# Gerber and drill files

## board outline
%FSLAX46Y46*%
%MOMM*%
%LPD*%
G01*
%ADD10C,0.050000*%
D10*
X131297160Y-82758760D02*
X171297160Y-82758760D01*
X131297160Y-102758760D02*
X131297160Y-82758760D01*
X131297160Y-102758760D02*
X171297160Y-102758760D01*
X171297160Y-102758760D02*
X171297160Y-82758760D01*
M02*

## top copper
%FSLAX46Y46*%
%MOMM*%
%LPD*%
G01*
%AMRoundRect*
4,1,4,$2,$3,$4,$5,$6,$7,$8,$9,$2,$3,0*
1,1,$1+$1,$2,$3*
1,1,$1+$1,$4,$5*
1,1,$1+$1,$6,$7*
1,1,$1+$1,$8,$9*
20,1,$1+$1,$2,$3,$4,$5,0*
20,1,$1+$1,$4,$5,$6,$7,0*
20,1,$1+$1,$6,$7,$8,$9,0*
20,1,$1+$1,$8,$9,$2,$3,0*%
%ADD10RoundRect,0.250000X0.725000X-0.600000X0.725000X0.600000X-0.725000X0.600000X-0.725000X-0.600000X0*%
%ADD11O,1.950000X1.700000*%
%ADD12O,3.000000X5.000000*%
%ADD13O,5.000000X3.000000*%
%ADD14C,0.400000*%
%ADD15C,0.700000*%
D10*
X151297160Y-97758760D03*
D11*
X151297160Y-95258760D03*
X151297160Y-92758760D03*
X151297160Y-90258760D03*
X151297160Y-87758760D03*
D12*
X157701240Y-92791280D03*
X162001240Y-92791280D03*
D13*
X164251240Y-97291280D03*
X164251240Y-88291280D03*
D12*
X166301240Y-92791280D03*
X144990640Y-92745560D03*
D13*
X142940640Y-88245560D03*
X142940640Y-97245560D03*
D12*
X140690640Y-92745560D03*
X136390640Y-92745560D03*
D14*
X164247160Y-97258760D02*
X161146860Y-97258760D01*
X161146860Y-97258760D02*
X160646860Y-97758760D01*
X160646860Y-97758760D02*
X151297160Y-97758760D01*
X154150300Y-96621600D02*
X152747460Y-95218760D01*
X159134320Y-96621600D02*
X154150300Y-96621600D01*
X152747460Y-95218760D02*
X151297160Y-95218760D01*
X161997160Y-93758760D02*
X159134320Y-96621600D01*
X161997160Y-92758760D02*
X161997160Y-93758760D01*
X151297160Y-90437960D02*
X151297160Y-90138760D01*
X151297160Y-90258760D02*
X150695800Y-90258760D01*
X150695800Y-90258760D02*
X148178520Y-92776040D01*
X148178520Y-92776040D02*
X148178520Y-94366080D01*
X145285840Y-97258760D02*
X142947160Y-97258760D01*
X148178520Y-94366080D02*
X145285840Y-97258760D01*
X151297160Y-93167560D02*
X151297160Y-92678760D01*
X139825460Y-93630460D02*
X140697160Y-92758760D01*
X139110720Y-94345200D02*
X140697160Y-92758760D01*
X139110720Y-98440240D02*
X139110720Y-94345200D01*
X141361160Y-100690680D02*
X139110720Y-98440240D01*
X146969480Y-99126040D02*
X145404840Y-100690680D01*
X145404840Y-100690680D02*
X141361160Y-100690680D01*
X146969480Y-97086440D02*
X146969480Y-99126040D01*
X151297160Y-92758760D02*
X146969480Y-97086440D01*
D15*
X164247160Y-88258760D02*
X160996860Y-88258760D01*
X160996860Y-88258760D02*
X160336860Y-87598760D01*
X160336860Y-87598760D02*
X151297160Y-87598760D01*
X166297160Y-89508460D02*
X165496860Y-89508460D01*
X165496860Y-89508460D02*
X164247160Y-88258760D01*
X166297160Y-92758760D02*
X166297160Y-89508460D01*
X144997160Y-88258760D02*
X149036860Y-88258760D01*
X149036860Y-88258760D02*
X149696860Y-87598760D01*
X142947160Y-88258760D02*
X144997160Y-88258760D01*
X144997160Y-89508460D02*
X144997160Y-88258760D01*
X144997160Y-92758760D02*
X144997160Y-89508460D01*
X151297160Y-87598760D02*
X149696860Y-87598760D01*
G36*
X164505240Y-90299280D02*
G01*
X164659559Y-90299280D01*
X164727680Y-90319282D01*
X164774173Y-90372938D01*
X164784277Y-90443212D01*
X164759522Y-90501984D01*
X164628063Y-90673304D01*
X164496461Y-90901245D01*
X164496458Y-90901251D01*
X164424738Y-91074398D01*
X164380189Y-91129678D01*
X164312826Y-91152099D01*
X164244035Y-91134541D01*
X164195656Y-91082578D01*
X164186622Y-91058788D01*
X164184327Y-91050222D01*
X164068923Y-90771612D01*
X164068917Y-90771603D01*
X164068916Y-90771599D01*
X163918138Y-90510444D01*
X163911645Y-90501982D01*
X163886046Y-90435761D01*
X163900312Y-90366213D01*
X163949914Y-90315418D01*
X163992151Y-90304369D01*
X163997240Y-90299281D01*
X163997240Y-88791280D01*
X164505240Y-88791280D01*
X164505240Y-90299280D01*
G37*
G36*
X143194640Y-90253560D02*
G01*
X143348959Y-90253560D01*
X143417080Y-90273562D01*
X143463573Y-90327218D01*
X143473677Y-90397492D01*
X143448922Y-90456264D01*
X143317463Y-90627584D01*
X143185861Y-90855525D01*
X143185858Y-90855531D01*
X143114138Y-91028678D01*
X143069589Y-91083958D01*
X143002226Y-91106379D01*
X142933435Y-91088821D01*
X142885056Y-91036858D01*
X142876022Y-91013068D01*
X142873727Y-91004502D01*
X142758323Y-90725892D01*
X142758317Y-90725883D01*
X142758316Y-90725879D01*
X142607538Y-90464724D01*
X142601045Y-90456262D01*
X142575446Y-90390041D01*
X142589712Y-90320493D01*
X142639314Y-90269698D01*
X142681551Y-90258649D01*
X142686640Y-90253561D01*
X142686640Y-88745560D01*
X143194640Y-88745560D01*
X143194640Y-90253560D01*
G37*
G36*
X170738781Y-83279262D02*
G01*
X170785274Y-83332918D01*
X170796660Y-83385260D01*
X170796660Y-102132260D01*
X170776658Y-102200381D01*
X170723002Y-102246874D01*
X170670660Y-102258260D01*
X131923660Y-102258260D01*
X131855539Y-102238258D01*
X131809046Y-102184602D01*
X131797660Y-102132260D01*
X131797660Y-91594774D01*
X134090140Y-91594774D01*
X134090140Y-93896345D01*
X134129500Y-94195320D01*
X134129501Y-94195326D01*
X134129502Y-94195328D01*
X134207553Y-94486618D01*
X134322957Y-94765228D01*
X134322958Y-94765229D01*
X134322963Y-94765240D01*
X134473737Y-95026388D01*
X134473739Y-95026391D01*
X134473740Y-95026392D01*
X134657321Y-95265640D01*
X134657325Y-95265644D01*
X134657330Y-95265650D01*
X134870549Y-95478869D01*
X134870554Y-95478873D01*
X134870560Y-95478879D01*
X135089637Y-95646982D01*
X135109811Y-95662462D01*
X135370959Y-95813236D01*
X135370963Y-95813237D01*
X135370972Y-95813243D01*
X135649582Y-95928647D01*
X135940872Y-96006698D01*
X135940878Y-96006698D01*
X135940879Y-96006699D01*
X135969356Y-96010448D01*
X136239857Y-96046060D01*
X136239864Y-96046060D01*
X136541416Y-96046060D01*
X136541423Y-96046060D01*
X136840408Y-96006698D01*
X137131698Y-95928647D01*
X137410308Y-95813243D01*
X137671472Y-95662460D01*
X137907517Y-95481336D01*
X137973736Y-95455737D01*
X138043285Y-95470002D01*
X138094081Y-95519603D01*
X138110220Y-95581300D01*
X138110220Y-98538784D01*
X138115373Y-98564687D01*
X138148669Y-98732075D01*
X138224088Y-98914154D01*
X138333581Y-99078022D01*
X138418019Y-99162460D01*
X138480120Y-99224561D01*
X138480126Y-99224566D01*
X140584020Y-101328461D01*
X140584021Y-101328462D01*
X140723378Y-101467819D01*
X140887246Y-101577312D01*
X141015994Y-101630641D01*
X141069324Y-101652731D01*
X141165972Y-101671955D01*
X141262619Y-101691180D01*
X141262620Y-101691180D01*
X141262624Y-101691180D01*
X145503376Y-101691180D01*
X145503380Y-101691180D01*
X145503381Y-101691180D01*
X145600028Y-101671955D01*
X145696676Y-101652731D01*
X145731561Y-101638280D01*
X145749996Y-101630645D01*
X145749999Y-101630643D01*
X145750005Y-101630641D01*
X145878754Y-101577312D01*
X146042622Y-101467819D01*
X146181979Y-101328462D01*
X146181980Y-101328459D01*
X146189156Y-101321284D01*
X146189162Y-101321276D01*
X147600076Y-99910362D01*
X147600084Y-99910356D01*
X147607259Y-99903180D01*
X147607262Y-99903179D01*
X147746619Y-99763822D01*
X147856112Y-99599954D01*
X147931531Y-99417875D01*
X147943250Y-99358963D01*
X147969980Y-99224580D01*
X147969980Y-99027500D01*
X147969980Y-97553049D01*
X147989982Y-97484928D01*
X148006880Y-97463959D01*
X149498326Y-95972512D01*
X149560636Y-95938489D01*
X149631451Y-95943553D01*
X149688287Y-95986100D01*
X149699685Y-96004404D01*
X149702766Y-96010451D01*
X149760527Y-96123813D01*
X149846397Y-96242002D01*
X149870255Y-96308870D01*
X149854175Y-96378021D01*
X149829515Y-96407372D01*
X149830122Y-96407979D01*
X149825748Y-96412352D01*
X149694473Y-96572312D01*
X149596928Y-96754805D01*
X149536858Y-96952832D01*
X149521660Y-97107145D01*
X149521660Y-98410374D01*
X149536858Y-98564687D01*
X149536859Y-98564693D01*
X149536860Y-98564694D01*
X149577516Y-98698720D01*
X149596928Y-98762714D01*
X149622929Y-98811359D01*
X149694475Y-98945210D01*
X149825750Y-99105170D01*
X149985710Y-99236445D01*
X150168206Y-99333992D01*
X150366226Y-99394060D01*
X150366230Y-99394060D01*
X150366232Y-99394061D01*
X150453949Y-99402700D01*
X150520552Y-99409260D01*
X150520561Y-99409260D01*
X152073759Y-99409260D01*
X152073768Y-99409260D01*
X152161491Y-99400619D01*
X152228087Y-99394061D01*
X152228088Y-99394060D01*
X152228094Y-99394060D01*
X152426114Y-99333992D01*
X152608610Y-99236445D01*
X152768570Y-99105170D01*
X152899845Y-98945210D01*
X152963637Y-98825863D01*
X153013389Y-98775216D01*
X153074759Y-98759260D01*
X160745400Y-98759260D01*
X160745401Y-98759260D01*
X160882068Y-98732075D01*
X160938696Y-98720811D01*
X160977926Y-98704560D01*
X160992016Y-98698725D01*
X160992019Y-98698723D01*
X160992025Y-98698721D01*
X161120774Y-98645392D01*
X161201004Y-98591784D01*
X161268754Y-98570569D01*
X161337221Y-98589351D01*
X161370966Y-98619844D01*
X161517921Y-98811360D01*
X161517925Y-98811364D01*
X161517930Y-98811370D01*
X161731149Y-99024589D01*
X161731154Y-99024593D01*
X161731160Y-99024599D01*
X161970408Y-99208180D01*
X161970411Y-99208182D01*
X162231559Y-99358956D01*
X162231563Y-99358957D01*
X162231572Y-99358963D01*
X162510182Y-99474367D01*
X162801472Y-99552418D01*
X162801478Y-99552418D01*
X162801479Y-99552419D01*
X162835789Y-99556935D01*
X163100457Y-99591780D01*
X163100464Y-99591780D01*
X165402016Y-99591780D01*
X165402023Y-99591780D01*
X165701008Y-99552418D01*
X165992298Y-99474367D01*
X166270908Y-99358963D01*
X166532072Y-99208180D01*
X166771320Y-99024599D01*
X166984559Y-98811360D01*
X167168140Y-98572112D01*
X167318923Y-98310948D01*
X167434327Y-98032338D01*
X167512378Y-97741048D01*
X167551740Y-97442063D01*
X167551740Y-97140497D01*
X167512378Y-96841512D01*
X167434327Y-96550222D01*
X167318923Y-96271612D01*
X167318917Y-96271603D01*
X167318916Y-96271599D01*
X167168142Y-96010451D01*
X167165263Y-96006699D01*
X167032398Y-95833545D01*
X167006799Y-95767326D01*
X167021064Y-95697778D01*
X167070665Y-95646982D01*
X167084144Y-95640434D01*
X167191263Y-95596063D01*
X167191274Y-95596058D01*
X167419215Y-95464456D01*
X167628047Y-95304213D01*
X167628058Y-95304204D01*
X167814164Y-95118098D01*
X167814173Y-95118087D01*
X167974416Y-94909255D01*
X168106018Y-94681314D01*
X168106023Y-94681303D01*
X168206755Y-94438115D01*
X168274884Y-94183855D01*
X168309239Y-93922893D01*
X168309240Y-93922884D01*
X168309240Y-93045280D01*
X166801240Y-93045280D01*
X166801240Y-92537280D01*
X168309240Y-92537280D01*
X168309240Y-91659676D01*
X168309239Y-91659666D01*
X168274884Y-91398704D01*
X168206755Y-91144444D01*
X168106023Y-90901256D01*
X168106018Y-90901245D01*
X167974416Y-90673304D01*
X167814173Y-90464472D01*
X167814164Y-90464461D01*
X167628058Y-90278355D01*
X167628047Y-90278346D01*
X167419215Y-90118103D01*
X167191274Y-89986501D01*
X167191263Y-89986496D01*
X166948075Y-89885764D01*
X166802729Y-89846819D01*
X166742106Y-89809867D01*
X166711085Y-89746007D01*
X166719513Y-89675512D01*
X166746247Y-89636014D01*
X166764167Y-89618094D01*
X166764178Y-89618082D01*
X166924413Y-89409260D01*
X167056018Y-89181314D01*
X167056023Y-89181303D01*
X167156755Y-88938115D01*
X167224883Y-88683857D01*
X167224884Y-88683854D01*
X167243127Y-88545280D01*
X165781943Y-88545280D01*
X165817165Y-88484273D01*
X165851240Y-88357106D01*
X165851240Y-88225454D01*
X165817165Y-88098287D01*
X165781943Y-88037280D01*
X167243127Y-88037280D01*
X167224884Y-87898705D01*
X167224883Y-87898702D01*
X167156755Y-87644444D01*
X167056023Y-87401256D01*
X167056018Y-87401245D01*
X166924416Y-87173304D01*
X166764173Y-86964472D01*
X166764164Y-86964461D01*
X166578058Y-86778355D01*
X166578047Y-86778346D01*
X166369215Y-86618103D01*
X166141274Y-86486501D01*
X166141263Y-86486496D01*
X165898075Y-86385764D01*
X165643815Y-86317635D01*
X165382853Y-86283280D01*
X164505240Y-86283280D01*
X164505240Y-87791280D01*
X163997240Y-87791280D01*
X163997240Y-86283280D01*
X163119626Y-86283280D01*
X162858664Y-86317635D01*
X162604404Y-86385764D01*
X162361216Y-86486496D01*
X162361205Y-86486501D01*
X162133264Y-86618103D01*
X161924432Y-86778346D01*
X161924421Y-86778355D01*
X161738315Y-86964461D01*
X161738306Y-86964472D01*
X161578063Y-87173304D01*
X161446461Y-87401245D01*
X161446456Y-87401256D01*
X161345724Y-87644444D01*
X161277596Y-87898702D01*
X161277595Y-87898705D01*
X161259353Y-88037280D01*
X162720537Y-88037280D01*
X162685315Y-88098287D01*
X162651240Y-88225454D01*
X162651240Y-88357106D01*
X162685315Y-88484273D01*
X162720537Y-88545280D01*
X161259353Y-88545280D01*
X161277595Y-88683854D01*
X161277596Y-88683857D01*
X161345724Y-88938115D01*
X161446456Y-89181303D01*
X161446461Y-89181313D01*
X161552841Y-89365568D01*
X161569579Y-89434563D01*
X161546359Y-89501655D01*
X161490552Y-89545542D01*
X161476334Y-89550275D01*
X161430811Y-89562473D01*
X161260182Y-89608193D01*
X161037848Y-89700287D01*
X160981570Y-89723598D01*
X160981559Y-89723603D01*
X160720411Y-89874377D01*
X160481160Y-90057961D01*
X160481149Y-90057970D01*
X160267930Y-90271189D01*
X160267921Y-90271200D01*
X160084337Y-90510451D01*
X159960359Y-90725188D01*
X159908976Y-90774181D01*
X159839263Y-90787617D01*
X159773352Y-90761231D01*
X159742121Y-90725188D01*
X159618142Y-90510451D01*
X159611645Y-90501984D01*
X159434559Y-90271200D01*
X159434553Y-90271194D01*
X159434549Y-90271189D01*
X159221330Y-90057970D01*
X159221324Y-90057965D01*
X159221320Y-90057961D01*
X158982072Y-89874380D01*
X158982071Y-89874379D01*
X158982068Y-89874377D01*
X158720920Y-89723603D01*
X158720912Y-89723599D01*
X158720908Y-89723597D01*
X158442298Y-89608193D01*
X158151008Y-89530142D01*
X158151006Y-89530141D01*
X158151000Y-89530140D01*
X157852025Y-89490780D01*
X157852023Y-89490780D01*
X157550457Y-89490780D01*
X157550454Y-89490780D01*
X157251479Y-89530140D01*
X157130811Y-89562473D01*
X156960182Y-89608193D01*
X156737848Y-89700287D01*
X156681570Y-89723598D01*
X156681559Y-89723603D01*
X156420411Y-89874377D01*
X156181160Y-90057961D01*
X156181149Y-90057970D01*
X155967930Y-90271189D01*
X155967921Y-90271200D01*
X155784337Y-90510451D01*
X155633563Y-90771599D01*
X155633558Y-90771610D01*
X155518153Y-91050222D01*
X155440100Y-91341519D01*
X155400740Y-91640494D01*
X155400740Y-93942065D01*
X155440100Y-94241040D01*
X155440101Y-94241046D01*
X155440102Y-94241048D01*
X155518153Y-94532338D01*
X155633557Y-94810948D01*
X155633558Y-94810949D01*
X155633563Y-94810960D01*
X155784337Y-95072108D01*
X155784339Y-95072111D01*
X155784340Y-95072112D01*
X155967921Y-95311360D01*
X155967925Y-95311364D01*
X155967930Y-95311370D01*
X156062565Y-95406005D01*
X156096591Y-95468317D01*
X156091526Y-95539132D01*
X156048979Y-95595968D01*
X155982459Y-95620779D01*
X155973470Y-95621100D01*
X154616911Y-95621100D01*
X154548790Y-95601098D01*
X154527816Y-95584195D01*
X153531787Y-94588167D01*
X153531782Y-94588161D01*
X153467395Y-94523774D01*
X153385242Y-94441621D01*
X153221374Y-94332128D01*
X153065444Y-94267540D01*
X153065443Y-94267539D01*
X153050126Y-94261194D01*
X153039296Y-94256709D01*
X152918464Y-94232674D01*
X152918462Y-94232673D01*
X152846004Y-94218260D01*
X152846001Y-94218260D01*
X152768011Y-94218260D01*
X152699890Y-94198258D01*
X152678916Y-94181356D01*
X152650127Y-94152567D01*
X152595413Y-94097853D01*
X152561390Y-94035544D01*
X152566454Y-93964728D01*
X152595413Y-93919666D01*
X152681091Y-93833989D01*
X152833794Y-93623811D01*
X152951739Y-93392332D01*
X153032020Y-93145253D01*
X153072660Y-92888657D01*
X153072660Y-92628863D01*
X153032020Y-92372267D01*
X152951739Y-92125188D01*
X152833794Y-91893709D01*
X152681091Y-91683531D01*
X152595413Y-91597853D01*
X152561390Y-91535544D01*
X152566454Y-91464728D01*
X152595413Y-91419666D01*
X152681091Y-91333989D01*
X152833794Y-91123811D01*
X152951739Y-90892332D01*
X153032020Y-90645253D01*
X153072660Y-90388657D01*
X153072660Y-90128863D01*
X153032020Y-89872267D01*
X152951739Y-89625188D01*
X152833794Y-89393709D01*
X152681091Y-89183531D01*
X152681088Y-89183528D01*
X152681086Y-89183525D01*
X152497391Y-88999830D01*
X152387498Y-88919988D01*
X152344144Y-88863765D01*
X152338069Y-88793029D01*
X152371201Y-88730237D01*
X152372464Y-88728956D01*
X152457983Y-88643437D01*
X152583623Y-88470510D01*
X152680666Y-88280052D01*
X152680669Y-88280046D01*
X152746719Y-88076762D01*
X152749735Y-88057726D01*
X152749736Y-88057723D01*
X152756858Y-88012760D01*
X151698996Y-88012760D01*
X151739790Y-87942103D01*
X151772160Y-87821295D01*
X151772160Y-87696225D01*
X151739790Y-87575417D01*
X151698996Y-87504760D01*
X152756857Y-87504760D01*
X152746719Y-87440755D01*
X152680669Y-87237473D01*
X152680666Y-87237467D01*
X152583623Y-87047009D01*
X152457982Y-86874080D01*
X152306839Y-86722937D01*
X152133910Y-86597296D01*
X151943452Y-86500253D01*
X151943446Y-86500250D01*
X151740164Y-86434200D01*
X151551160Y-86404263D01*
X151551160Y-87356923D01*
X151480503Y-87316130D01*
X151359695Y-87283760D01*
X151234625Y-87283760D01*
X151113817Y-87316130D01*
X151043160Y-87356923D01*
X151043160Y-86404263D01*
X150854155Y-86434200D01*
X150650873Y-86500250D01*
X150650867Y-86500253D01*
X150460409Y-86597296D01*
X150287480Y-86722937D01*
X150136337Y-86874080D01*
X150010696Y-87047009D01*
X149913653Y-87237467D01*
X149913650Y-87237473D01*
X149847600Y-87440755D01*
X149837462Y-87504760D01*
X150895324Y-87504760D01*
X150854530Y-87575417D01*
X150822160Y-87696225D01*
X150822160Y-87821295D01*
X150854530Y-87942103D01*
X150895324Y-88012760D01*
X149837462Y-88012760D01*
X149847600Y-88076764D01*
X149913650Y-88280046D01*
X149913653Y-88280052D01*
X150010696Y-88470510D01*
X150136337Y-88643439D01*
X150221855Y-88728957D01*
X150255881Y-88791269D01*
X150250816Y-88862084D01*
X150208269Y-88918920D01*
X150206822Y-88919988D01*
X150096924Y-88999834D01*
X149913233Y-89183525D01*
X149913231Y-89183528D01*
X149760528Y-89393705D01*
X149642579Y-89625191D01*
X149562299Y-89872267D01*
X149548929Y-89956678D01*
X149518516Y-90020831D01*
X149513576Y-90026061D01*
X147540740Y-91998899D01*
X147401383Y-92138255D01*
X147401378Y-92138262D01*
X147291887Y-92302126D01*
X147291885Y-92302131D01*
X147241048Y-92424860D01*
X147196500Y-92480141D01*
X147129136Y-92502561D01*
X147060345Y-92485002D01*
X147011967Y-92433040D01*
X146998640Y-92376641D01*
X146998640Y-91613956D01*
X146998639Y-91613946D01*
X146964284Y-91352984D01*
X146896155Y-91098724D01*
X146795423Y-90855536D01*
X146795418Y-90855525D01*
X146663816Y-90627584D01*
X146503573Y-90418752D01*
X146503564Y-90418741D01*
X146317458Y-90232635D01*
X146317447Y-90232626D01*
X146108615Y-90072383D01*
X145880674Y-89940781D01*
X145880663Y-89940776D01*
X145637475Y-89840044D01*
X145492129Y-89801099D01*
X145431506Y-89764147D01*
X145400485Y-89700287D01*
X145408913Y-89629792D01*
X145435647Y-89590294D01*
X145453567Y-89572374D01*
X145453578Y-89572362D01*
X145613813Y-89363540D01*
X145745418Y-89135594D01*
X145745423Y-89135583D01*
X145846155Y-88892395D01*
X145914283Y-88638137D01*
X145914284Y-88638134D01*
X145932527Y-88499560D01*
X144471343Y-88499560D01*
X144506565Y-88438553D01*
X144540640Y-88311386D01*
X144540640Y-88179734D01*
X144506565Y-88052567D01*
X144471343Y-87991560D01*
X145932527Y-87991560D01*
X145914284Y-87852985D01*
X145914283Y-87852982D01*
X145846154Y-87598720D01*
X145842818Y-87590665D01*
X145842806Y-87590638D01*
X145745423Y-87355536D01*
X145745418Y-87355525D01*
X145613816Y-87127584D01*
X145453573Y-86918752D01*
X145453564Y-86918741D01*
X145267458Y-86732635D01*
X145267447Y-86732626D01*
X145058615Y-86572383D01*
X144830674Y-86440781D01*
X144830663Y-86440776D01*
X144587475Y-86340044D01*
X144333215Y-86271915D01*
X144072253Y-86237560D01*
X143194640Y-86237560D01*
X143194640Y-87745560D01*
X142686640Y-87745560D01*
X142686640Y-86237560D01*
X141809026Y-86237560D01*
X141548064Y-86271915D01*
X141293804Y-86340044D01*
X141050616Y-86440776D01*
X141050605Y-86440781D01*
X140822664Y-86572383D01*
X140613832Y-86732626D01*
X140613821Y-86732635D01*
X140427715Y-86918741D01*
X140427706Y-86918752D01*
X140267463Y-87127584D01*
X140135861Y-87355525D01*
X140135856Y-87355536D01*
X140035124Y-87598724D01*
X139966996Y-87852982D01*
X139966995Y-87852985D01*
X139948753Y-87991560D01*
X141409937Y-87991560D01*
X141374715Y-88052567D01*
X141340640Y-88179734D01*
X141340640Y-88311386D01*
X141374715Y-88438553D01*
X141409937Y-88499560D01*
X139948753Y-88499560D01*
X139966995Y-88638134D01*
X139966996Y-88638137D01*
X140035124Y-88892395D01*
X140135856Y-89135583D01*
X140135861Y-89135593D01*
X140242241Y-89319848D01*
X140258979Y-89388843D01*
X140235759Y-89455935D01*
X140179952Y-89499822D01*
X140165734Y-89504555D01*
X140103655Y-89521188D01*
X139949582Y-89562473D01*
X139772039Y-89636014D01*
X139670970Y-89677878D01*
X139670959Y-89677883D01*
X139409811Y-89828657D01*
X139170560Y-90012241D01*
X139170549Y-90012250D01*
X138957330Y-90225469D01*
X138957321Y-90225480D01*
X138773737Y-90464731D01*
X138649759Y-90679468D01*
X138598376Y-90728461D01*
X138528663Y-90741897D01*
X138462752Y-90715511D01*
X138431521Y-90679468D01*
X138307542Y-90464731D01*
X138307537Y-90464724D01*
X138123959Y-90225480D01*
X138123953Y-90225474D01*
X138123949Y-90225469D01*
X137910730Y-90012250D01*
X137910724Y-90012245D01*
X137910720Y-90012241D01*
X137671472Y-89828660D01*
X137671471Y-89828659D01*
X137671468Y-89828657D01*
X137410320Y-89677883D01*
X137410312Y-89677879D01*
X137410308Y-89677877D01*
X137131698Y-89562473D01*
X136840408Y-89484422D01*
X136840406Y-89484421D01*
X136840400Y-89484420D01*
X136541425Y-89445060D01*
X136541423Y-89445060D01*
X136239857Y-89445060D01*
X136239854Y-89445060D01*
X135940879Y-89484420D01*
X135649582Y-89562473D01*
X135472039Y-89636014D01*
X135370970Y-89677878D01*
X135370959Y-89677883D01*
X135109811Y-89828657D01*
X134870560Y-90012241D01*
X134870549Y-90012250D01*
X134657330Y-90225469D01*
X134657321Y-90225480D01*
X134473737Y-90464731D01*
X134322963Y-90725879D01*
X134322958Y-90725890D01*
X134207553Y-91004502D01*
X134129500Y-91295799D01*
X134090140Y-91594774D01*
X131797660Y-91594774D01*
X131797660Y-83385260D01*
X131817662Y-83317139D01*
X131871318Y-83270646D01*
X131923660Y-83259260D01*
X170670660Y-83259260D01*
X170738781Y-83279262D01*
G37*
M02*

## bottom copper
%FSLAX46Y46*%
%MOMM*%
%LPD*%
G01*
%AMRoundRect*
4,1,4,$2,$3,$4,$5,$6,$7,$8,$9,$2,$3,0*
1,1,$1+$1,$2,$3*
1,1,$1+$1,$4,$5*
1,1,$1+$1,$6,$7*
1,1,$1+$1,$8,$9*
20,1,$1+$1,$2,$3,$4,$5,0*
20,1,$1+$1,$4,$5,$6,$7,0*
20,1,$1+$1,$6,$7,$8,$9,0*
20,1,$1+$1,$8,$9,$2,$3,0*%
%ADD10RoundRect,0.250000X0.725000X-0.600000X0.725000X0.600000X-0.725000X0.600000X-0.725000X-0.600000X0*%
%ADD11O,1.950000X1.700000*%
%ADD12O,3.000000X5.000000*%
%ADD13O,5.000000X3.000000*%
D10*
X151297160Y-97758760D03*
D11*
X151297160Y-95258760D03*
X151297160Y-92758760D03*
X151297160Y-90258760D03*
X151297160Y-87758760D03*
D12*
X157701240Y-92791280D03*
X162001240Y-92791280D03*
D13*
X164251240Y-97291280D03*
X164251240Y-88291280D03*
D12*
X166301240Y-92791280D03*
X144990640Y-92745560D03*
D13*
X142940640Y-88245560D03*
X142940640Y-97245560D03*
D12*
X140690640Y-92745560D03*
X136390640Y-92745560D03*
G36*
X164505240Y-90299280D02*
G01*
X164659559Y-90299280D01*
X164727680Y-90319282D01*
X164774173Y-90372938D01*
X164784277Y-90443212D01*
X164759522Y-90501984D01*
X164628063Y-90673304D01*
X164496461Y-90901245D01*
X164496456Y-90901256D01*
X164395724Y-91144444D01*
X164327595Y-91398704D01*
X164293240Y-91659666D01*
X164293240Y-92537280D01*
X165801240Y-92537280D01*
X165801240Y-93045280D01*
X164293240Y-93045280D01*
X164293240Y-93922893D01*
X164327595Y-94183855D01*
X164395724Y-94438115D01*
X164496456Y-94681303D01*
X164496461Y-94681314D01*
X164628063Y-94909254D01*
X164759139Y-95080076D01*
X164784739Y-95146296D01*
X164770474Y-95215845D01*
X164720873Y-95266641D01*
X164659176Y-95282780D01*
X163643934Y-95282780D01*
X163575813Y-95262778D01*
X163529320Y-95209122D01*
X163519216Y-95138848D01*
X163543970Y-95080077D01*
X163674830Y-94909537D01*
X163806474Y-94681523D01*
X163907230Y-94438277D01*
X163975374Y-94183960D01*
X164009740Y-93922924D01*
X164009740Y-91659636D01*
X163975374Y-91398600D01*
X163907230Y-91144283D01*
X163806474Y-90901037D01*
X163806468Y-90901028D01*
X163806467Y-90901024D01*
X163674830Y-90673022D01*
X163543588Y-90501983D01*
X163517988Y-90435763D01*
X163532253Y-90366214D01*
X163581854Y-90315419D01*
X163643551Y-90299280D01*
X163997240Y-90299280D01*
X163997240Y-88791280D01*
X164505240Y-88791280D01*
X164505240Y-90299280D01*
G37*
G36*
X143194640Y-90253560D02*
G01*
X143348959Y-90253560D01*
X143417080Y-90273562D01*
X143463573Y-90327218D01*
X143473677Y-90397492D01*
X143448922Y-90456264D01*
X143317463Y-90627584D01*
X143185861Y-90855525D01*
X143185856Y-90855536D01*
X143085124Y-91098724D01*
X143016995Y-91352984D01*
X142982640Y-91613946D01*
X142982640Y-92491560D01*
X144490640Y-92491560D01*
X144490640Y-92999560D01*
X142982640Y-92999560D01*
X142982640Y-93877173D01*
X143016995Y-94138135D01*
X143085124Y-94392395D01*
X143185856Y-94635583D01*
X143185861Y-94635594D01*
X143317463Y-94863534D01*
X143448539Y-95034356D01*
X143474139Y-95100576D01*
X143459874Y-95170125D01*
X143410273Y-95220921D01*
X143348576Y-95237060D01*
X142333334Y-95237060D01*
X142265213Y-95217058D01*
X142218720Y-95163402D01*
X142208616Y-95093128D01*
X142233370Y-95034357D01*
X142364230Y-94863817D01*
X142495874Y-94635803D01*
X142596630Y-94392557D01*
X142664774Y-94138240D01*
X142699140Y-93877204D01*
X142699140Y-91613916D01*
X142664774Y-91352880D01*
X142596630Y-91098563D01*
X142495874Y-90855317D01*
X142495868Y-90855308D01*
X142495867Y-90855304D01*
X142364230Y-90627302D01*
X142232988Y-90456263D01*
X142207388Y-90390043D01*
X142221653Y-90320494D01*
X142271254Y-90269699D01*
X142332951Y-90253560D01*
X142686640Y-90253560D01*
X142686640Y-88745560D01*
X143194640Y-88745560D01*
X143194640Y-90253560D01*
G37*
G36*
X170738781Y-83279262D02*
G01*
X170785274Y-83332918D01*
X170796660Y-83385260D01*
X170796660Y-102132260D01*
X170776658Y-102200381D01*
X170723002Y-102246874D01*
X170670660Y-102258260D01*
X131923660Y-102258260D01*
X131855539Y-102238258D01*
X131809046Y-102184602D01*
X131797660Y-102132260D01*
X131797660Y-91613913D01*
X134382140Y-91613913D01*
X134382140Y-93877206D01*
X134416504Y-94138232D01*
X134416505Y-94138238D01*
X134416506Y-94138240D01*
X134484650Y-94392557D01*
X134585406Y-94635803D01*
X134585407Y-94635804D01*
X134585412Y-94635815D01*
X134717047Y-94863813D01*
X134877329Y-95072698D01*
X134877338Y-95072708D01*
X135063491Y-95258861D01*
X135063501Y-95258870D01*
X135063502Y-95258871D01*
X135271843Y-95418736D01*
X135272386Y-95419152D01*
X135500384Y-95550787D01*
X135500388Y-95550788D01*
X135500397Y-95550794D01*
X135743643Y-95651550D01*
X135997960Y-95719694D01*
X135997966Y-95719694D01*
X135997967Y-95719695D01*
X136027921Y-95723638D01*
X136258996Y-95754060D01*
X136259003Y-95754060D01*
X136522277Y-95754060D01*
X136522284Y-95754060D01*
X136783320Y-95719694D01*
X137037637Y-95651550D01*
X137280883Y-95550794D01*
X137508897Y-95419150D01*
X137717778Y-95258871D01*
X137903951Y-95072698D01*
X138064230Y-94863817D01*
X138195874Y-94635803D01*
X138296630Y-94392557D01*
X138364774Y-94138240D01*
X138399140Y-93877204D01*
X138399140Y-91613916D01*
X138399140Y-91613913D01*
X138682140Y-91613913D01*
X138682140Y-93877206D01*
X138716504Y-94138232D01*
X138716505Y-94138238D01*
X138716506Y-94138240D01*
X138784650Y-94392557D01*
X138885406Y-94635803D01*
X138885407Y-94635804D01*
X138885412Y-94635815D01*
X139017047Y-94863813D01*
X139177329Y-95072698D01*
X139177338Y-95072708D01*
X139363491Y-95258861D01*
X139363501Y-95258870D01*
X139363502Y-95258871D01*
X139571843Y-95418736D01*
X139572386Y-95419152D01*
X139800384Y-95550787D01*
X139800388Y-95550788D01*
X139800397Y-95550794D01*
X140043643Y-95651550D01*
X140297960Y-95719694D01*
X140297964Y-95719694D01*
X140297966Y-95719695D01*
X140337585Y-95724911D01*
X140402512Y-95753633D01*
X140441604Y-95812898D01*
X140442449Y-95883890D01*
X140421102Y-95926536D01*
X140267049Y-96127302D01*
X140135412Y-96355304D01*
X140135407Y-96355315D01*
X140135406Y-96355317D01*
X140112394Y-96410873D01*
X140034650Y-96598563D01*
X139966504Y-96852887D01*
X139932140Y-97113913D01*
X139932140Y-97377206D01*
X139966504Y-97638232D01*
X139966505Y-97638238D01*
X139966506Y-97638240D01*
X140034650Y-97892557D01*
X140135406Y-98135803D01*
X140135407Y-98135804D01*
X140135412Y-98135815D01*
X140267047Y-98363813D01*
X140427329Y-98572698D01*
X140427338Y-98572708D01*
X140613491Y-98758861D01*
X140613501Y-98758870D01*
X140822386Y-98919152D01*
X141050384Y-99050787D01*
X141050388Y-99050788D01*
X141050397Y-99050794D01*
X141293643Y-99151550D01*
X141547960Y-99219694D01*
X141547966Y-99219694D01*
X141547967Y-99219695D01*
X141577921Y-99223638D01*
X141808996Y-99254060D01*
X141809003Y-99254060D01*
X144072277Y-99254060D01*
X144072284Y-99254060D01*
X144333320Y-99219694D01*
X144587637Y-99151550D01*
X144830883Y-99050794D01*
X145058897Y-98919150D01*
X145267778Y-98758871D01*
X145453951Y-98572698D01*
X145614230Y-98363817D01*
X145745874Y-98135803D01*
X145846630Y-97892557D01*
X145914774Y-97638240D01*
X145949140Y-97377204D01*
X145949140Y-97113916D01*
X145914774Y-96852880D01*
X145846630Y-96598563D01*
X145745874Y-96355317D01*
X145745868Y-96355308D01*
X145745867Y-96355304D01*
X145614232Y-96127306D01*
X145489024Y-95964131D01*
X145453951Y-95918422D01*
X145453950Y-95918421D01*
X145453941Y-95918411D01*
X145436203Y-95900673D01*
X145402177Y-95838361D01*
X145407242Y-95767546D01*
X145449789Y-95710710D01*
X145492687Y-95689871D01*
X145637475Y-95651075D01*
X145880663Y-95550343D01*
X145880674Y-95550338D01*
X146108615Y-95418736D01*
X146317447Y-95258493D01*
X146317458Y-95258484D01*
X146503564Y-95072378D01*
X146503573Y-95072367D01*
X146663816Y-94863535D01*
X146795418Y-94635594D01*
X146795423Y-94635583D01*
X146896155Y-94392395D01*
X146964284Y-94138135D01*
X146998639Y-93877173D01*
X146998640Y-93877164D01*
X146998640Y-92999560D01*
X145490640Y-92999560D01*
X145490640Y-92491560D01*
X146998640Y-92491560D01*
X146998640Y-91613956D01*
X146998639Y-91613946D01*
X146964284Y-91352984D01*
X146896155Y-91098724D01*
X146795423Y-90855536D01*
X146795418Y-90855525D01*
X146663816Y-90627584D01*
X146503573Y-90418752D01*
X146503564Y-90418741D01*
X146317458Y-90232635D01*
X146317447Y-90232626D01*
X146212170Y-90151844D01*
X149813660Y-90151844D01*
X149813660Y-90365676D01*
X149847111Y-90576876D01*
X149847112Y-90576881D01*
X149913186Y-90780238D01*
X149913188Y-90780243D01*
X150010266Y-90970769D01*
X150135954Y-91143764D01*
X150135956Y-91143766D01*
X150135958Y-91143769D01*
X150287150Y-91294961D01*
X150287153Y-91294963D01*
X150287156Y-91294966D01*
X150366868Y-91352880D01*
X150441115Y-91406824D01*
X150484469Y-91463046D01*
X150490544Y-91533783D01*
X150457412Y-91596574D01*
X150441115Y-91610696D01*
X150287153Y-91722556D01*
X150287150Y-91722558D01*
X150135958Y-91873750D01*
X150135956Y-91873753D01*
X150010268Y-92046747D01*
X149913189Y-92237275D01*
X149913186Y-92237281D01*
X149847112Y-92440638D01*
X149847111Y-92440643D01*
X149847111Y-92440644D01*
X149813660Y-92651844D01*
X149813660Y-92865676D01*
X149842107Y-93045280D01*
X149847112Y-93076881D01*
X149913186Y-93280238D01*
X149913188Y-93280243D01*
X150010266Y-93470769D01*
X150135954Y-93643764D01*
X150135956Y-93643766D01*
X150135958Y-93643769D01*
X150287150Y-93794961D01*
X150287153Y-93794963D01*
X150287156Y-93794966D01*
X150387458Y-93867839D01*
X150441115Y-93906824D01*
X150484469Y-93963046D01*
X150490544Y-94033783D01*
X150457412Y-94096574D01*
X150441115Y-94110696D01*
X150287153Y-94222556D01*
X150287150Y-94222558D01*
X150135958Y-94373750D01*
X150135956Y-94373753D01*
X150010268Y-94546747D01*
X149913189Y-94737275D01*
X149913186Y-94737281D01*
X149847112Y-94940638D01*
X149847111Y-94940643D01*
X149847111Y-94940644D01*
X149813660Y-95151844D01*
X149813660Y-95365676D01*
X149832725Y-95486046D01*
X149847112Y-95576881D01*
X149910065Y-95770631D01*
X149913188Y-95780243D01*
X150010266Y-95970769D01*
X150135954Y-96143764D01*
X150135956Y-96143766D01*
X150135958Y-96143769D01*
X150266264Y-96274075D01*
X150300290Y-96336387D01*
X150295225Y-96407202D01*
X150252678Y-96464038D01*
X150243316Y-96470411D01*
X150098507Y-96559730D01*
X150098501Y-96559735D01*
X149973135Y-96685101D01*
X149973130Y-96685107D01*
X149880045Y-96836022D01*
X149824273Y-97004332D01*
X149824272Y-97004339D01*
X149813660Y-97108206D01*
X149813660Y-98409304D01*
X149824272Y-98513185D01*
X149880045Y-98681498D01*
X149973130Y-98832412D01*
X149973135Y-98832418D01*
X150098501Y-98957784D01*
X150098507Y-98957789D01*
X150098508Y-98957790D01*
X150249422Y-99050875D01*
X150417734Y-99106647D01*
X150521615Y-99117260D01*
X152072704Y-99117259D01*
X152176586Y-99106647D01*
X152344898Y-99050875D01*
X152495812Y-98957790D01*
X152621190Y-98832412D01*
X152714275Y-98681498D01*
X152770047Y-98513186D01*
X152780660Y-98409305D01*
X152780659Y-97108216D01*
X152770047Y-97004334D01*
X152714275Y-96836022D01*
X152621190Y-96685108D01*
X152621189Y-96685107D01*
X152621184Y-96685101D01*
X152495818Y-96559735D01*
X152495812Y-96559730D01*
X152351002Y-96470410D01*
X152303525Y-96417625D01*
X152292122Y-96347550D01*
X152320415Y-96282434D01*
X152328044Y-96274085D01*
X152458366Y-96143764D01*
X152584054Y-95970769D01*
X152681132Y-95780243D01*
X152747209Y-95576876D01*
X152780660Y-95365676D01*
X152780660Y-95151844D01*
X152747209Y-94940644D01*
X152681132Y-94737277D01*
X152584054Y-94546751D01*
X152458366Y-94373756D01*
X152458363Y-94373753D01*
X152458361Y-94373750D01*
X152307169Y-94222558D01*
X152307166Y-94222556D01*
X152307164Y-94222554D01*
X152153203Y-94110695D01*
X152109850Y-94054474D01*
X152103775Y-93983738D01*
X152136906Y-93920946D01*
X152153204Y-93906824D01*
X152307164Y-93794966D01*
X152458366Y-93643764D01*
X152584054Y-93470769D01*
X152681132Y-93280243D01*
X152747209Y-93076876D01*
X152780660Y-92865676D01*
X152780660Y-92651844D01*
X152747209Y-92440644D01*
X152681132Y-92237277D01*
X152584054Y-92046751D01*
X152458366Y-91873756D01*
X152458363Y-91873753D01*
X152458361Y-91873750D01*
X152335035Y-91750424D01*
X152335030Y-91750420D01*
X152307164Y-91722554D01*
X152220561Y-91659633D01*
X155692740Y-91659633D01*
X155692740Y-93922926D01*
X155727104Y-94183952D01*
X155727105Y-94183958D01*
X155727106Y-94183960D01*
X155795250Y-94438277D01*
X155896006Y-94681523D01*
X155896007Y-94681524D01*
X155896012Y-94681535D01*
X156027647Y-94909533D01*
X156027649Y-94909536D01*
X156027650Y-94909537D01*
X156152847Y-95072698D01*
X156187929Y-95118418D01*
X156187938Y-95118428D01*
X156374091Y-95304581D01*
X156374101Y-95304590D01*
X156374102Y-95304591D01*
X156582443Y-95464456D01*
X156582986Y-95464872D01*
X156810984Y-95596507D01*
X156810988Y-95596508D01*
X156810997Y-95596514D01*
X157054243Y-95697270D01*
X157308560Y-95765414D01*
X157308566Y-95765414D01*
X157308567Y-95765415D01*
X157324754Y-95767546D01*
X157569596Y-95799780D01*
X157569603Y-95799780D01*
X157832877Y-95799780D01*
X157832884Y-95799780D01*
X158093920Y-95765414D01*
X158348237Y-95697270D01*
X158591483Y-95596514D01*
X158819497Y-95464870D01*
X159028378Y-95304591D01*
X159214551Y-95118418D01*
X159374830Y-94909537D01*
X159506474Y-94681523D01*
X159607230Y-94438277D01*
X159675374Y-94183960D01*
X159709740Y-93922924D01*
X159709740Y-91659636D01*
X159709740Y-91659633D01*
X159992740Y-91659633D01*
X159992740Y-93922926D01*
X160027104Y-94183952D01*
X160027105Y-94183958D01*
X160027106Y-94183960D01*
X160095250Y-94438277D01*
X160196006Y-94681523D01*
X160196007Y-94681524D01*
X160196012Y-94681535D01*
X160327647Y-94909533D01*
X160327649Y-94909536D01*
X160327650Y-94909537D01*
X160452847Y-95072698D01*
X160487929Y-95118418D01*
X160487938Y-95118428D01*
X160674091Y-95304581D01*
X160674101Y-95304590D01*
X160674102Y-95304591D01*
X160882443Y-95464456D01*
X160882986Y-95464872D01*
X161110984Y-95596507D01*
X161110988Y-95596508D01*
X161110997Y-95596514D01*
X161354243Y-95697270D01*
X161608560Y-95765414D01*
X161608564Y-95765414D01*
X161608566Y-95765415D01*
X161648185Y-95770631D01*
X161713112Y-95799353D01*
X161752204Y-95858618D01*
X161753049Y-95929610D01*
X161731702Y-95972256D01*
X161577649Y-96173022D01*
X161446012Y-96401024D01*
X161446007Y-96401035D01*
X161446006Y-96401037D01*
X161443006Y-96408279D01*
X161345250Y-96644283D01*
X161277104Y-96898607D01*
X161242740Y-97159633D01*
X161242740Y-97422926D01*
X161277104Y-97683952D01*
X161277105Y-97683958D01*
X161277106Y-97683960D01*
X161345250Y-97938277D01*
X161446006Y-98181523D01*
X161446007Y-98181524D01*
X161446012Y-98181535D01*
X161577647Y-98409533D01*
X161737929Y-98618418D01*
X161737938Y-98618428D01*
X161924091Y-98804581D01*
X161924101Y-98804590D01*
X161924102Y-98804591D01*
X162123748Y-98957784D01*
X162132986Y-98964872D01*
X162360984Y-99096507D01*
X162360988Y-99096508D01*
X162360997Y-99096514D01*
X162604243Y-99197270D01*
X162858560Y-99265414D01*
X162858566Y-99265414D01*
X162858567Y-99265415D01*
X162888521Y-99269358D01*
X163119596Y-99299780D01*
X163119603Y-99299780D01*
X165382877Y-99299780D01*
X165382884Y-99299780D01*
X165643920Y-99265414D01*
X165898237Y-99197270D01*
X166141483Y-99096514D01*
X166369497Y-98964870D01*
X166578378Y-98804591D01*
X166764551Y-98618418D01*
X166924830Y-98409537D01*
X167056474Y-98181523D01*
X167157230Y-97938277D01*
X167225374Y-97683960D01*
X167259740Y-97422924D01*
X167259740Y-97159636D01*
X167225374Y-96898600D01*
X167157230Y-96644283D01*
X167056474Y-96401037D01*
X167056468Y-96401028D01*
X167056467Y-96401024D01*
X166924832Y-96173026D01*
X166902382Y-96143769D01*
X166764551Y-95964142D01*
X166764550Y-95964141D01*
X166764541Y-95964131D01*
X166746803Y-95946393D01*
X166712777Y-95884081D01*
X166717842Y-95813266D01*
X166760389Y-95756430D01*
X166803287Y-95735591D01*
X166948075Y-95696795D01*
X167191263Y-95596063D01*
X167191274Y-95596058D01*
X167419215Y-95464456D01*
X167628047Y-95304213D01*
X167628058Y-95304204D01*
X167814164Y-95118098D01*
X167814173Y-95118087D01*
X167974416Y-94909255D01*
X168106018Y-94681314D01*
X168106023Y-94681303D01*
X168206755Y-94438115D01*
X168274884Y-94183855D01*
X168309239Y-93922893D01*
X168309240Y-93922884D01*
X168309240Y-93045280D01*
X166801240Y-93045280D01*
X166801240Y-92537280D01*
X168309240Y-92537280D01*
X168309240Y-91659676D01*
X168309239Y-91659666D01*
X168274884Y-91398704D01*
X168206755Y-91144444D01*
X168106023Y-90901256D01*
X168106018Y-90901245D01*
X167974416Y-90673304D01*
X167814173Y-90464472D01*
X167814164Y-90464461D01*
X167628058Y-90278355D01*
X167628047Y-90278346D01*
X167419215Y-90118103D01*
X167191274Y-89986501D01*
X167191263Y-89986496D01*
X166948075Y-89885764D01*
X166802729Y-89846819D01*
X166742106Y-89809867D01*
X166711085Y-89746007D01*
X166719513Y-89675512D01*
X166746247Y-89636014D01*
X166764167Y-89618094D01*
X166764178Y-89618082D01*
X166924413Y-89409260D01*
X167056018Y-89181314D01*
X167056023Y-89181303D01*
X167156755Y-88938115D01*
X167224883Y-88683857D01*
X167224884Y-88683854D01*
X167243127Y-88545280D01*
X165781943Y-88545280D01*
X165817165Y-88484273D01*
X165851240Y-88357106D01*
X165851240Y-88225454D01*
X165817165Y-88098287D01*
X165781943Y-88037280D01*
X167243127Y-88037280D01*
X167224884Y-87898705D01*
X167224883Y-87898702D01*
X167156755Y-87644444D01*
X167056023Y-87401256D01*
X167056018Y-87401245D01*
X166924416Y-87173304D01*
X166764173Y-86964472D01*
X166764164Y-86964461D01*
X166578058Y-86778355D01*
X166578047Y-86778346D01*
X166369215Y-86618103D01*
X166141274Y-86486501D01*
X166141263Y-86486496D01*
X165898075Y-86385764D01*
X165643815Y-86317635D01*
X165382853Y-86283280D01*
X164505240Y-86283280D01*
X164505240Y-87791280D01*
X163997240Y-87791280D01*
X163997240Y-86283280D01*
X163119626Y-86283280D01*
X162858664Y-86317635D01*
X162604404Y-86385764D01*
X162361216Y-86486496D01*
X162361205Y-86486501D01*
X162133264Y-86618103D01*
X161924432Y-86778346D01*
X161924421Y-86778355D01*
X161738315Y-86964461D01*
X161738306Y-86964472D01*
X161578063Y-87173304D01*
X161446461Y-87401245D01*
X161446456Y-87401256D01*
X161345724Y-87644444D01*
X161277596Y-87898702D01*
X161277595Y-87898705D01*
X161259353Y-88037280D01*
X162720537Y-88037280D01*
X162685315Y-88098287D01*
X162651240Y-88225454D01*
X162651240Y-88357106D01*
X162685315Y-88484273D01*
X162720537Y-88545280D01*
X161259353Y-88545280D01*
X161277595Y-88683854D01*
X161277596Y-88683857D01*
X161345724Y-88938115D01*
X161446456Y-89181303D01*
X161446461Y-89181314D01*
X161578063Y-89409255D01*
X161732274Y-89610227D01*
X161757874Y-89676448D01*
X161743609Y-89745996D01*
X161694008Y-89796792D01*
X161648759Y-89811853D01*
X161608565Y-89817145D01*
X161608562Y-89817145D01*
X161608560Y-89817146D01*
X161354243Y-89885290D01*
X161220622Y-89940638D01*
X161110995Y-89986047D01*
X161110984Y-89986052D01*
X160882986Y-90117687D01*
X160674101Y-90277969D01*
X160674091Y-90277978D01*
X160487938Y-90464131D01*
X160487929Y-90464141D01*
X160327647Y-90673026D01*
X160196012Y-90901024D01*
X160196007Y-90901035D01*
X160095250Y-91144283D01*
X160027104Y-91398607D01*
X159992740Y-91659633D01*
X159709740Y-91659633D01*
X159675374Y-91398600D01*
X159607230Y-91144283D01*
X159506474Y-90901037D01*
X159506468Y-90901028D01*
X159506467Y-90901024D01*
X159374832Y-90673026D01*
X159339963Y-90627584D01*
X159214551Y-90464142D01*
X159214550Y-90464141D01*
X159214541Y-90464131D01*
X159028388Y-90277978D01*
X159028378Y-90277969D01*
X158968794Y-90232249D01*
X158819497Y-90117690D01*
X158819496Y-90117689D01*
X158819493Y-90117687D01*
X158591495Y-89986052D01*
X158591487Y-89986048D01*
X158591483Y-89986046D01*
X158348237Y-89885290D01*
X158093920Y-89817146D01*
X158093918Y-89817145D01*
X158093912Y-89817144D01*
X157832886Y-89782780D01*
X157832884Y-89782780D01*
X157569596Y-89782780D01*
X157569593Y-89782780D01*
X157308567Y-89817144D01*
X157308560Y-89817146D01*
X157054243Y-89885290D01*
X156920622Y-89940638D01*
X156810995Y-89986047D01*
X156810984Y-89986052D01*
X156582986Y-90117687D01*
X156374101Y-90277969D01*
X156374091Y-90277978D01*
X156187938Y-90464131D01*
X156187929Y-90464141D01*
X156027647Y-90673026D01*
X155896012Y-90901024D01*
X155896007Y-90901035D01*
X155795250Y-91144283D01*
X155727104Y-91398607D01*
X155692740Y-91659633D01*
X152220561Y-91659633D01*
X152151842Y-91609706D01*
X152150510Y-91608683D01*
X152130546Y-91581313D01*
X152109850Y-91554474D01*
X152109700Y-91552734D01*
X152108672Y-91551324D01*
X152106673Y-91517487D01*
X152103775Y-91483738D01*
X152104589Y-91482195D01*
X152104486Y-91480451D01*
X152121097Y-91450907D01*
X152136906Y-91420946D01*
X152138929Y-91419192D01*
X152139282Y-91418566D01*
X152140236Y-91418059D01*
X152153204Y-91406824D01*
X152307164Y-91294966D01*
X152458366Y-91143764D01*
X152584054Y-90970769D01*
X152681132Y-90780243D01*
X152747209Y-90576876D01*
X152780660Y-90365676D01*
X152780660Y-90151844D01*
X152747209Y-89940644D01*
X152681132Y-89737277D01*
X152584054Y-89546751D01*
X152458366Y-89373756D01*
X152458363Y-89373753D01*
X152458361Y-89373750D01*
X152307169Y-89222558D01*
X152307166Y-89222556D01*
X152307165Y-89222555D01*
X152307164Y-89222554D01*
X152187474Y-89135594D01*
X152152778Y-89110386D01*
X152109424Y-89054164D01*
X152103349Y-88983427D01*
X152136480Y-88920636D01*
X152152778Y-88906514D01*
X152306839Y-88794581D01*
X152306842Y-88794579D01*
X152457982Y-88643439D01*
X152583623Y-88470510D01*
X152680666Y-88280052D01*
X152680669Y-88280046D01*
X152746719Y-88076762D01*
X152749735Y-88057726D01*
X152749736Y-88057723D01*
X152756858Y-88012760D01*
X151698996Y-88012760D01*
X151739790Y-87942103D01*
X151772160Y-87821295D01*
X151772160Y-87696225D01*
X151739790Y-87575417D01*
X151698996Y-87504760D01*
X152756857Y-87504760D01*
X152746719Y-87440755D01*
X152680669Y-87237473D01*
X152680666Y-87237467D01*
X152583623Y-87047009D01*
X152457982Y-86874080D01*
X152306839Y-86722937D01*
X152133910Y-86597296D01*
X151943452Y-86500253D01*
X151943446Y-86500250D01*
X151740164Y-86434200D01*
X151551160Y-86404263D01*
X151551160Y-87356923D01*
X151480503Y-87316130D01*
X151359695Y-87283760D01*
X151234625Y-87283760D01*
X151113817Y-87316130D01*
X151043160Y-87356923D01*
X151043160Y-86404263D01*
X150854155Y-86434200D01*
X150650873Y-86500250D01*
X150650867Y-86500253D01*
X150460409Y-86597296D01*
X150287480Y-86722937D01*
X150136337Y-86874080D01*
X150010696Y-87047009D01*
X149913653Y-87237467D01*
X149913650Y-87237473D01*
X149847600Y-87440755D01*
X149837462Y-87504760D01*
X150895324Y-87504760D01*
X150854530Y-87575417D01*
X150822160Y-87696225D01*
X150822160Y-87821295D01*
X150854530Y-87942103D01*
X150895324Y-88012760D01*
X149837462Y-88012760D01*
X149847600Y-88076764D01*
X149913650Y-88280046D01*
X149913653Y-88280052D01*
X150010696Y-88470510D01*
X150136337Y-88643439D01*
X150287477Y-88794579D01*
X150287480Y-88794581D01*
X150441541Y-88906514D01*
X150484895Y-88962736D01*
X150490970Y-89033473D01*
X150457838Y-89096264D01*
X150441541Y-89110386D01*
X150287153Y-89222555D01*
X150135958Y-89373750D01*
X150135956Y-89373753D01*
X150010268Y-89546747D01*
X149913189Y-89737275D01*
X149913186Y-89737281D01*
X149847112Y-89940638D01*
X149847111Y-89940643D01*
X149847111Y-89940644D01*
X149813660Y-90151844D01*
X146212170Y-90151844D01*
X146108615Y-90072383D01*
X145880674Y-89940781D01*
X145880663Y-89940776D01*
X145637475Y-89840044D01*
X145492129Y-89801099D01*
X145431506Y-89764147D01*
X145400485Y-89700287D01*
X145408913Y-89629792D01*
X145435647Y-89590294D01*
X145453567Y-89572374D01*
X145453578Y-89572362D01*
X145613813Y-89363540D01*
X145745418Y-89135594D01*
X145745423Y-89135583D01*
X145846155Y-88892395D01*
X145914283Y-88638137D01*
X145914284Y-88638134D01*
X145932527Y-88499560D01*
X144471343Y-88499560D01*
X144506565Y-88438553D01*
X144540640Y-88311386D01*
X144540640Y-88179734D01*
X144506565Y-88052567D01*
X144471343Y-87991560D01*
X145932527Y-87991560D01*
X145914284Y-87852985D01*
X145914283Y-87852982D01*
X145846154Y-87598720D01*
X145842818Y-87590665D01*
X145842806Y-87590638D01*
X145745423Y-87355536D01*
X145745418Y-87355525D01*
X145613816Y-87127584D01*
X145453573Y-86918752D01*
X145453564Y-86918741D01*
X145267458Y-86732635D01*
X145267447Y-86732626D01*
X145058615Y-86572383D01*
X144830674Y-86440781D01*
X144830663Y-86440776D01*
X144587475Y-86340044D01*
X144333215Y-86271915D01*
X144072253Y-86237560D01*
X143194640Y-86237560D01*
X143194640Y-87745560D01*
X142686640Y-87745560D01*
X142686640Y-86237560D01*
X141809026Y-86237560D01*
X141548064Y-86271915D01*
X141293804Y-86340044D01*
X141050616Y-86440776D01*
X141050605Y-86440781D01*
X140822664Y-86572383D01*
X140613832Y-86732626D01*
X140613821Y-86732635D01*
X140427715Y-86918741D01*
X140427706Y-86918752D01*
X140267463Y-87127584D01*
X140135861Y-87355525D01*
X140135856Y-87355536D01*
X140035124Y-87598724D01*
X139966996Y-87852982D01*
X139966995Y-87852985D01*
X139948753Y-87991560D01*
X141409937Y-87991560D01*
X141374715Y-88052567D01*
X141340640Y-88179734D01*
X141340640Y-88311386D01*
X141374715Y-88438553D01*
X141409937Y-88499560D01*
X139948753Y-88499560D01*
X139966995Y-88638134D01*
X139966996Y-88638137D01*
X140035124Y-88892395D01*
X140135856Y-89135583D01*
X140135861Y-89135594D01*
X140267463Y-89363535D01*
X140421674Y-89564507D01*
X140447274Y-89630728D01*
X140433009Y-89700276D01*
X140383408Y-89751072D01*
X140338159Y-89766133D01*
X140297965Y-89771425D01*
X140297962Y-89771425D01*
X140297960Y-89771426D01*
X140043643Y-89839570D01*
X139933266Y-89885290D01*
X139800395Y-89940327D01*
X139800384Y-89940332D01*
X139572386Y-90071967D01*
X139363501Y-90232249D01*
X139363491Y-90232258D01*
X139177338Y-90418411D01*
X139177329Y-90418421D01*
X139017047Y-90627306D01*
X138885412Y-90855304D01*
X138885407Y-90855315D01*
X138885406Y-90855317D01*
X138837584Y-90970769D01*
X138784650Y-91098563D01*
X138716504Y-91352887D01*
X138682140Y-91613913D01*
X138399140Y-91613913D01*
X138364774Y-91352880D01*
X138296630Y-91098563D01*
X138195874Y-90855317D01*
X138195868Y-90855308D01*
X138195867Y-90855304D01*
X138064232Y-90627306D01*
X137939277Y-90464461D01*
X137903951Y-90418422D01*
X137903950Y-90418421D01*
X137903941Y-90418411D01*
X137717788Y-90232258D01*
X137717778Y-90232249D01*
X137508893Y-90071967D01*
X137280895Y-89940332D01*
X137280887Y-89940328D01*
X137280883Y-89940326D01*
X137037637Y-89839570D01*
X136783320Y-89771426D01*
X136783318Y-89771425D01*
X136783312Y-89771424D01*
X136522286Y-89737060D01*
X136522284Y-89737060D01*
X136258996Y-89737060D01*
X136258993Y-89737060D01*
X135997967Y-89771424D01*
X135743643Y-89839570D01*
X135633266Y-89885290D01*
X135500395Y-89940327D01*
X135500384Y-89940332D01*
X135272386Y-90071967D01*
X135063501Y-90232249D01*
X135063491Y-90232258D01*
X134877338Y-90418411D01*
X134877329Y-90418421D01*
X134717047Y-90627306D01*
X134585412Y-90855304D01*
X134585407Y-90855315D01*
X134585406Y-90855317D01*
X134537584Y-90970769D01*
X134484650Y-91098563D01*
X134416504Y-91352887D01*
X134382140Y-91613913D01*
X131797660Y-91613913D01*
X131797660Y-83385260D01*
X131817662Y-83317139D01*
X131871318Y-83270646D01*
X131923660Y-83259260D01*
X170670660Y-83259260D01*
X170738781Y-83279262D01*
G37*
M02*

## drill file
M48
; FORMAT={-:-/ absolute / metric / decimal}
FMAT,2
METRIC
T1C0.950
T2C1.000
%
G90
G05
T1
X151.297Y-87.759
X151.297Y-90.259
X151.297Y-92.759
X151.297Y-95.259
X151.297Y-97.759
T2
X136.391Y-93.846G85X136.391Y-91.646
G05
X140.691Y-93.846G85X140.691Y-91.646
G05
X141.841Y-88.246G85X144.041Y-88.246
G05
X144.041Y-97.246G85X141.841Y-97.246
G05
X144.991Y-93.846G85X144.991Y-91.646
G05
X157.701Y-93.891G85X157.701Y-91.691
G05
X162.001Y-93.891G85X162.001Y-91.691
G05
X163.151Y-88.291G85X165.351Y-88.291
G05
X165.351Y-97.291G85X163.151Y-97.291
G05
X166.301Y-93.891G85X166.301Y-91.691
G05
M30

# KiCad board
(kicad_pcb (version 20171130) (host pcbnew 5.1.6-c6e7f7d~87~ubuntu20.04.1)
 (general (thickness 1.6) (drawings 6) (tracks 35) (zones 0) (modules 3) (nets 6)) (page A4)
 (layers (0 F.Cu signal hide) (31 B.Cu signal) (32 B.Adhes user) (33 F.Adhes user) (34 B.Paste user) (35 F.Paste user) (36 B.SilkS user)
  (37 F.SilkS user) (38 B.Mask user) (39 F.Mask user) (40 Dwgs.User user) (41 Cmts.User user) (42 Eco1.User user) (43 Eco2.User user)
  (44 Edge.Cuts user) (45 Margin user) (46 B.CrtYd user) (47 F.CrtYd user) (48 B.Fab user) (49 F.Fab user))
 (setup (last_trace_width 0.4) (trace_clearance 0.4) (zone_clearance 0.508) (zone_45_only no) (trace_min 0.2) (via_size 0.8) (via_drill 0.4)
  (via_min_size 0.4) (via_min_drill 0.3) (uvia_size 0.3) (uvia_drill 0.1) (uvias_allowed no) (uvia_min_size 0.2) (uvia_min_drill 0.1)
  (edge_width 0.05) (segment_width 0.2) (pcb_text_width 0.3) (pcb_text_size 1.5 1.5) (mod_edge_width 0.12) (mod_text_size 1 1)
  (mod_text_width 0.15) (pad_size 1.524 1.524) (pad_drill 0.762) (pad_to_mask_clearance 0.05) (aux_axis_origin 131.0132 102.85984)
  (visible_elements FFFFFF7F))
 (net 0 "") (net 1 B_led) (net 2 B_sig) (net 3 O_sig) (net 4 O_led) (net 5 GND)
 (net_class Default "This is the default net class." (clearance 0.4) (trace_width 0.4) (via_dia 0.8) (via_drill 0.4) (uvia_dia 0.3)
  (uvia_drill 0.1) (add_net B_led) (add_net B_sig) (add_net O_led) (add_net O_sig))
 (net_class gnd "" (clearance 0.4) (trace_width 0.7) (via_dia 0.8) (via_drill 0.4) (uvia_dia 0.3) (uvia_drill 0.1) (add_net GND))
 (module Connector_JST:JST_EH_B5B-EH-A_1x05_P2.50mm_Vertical (layer F.Cu) (at 151.29716 97.75876 90)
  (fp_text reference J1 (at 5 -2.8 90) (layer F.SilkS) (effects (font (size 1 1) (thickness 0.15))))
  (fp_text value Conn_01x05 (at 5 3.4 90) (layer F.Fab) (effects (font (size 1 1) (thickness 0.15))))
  (pad 1 thru_hole roundrect (at 0 0 90) (size 1.7 1.95) (drill 0.95) (layers *.Cu *.Mask) (roundrect_rratio 0.147059) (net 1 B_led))
  (pad 2 thru_hole oval (at 2.5 0 90) (size 1.7 1.95) (drill 0.95) (layers *.Cu *.Mask) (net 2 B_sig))
  (pad 3 thru_hole oval (at 5 0 90) (size 1.7 1.95) (drill 0.95) (layers *.Cu *.Mask) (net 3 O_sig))
  (pad 4 thru_hole oval (at 7.5 0 90) (size 1.7 1.95) (drill 0.95) (layers *.Cu *.Mask) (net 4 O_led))
  (pad 5 thru_hole oval (at 10 0 90) (size 1.7 1.95) (drill 0.95) (layers *.Cu *.Mask) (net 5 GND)))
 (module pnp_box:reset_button (layer F.Cu) (at 154.70124 92.79128 90)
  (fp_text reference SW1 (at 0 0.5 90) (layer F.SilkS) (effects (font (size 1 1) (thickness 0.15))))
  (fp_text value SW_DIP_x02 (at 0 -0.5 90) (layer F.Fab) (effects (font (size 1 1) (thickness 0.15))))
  (pad 0 thru_hole oval (at 0 3 90) (size 5 3) (drill oval 3.2 1) (layers *.Cu *.Mask))
  (pad 2 thru_hole oval (at 0 7.3 90) (size 5 3) (drill oval 3.2 1) (layers *.Cu *.Mask) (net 2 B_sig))
  (pad 1 thru_hole oval (at -4.5 9.55 180) (size 5 3) (drill oval 3.2 1) (layers *.Cu *.Mask) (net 1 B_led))
  (pad 4 thru_hole oval (at 4.5 9.55) (size 5 3) (drill oval 3.2 1) (layers *.Cu *.Mask) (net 5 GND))
  (pad 3 thru_hole oval (at 0 11.6 90) (size 5 3) (drill oval 3.2 1) (layers *.Cu *.Mask) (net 5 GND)))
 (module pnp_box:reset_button (layer F.Cu) (at 133.39064 92.74556 90)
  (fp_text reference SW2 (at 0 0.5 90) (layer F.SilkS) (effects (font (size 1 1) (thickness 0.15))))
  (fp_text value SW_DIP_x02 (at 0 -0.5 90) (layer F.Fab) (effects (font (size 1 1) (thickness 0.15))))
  (pad 3 thru_hole oval (at 0 11.6 90) (size 5 3) (drill oval 3.2 1) (layers *.Cu *.Mask) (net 5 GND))
  (pad 4 thru_hole oval (at 4.5 9.55) (size 5 3) (drill oval 3.2 1) (layers *.Cu *.Mask) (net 5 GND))
  (pad 1 thru_hole oval (at -4.5 9.55 180) (size 5 3) (drill oval 3.2 1) (layers *.Cu *.Mask) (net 4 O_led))
  (pad 2 thru_hole oval (at 0 7.3 90) (size 5 3) (drill oval 3.2 1) (layers *.Cu *.Mask) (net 3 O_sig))
  (pad 0 thru_hole oval (at 0 3 90) (size 5 3) (drill oval 3.2 1) (layers *.Cu *.Mask)))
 (gr_line (start 131.29716 82.75876) (end 171.29716 82.75876) (layer Edge.Cuts) (width 0.05))
 (gr_line (start 131.29716 102.75876) (end 131.29716 82.75876) (layer Edge.Cuts) (width 0.05))
 (gr_line (start 131.29716 102.75876) (end 171.29716 102.75876) (layer Edge.Cuts) (width 0.05))
 (gr_line (start 171.29716 102.75876) (end 171.29716 82.75876) (layer Edge.Cuts) (width 0.05))
 (segment (start 164.24716 97.25876) (end 161.14686 97.25876) (width 0.4) (layer F.Cu) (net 1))
 (segment (start 161.14686 97.25876) (end 160.64686 97.75876) (width 0.4) (layer F.Cu) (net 1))
 (segment (start 160.64686 97.75876) (end 151.29716 97.75876) (width 0.4) (layer F.Cu) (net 1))
 (segment (start 154.1503 96.6216) (end 152.74746 95.21876) (width 0.4) (layer F.Cu) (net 2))
 (segment (start 159.13432 96.6216) (end 154.1503 96.6216) (width 0.4) (layer F.Cu) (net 2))
 (segment (start 152.74746 95.21876) (end 151.29716 95.21876) (width 0.4) (layer F.Cu) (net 2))
 (segment (start 161.99716 93.75876) (end 159.13432 96.6216) (width 0.4) (layer F.Cu) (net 2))
 (segment (start 161.99716 92.75876) (end 161.99716 93.75876) (width 0.4) (layer F.Cu) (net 2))
 (segment (start 151.29716 90.43796) (end 151.29716 90.13876) (width 0.4) (layer F.Cu) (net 4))
 (segment (start 151.29716 90.25876) (end 150.6958 90.25876) (width 0.4) (layer F.Cu) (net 4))
 (segment (start 150.6958 90.25876) (end 148.17852 92.77604) (width 0.4) (layer F.Cu) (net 4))
 (segment (start 148.17852 92.77604) (end 148.17852 94.36608) (width 0.4) (layer F.Cu) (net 4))
 (segment (start 145.28584 97.25876) (end 142.94716 97.25876) (width 0.4) (layer F.Cu) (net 4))
 (segment (start 148.17852 94.36608) (end 145.28584 97.25876) (width 0.4) (layer F.Cu) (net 4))
 (segment (start 151.29716 93.16756) (end 151.29716 92.67876) (width 0.4) (layer F.Cu) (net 3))
 (segment (start 139.82546 93.63046) (end 140.69716 92.75876) (width 0.4) (layer F.Cu) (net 3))
 (segment (start 139.11072 94.3452) (end 140.69716 92.75876) (width 0.4) (layer F.Cu) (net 3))
 (segment (start 139.11072 98.44024) (end 139.11072 94.3452) (width 0.4) (layer F.Cu) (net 3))
 (segment (start 141.36116 100.69068) (end 139.11072 98.44024) (width 0.4) (layer F.Cu) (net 3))
 (segment (start 146.96948 99.12604) (end 145.40484 100.69068) (width 0.4) (layer F.Cu) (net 3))
 (segment (start 145.40484 100.69068) (end 141.36116 100.69068) (width 0.4) (layer F.Cu) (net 3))
 (segment (start 146.96948 97.08644) (end 146.96948 99.12604) (width 0.4) (layer F.Cu) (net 3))
 (segment (start 151.29716 92.75876) (end 146.96948 97.08644) (width 0.4) (layer F.Cu) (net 3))
 (segment (start 164.24716 88.25876) (end 160.99686 88.25876) (width 0.7) (layer F.Cu) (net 5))
 (segment (start 160.99686 88.25876) (end 160.33686 87.59876) (width 0.7) (layer F.Cu) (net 5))
 (segment (start 160.33686 87.59876) (end 151.29716 87.59876) (width 0.7) (layer F.Cu) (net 5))
 (segment (start 166.29716 89.50846) (end 165.49686 89.50846) (width 0.7) (layer F.Cu) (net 5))
 (segment (start 165.49686 89.50846) (end 164.24716 88.25876) (width 0.7) (layer F.Cu) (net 5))
 (segment (start 166.29716 92.75876) (end 166.29716 89.50846) (width 0.7) (layer F.Cu) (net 5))
 (segment (start 144.99716 88.25876) (end 149.03686 88.25876) (width 0.7) (layer F.Cu) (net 5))
 (segment (start 149.03686 88.25876) (end 149.69686 87.59876) (width 0.7) (layer F.Cu) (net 5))
 (segment (start 142.94716 88.25876) (end 144.99716 88.25876) (width 0.7) (layer F.Cu) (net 5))
 (segment (start 144.99716 89.50846) (end 144.99716 88.25876) (width 0.7) (layer F.Cu) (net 5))
 (segment (start 144.99716 92.75876) (end 144.99716 89.50846) (width 0.7) (layer F.Cu) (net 5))
 (segment (start 151.29716 87.59876) (end 149.69686 87.59876) (width 0.7) (layer F.Cu) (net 5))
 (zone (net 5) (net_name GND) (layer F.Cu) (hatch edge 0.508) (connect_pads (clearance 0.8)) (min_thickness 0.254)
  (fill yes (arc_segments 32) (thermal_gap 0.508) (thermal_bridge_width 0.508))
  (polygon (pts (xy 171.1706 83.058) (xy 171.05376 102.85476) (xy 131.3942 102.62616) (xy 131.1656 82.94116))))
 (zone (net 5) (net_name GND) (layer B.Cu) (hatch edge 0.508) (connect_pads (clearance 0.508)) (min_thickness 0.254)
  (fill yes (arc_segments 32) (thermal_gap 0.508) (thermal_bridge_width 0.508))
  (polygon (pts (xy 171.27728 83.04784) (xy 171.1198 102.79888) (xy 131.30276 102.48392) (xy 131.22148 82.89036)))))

